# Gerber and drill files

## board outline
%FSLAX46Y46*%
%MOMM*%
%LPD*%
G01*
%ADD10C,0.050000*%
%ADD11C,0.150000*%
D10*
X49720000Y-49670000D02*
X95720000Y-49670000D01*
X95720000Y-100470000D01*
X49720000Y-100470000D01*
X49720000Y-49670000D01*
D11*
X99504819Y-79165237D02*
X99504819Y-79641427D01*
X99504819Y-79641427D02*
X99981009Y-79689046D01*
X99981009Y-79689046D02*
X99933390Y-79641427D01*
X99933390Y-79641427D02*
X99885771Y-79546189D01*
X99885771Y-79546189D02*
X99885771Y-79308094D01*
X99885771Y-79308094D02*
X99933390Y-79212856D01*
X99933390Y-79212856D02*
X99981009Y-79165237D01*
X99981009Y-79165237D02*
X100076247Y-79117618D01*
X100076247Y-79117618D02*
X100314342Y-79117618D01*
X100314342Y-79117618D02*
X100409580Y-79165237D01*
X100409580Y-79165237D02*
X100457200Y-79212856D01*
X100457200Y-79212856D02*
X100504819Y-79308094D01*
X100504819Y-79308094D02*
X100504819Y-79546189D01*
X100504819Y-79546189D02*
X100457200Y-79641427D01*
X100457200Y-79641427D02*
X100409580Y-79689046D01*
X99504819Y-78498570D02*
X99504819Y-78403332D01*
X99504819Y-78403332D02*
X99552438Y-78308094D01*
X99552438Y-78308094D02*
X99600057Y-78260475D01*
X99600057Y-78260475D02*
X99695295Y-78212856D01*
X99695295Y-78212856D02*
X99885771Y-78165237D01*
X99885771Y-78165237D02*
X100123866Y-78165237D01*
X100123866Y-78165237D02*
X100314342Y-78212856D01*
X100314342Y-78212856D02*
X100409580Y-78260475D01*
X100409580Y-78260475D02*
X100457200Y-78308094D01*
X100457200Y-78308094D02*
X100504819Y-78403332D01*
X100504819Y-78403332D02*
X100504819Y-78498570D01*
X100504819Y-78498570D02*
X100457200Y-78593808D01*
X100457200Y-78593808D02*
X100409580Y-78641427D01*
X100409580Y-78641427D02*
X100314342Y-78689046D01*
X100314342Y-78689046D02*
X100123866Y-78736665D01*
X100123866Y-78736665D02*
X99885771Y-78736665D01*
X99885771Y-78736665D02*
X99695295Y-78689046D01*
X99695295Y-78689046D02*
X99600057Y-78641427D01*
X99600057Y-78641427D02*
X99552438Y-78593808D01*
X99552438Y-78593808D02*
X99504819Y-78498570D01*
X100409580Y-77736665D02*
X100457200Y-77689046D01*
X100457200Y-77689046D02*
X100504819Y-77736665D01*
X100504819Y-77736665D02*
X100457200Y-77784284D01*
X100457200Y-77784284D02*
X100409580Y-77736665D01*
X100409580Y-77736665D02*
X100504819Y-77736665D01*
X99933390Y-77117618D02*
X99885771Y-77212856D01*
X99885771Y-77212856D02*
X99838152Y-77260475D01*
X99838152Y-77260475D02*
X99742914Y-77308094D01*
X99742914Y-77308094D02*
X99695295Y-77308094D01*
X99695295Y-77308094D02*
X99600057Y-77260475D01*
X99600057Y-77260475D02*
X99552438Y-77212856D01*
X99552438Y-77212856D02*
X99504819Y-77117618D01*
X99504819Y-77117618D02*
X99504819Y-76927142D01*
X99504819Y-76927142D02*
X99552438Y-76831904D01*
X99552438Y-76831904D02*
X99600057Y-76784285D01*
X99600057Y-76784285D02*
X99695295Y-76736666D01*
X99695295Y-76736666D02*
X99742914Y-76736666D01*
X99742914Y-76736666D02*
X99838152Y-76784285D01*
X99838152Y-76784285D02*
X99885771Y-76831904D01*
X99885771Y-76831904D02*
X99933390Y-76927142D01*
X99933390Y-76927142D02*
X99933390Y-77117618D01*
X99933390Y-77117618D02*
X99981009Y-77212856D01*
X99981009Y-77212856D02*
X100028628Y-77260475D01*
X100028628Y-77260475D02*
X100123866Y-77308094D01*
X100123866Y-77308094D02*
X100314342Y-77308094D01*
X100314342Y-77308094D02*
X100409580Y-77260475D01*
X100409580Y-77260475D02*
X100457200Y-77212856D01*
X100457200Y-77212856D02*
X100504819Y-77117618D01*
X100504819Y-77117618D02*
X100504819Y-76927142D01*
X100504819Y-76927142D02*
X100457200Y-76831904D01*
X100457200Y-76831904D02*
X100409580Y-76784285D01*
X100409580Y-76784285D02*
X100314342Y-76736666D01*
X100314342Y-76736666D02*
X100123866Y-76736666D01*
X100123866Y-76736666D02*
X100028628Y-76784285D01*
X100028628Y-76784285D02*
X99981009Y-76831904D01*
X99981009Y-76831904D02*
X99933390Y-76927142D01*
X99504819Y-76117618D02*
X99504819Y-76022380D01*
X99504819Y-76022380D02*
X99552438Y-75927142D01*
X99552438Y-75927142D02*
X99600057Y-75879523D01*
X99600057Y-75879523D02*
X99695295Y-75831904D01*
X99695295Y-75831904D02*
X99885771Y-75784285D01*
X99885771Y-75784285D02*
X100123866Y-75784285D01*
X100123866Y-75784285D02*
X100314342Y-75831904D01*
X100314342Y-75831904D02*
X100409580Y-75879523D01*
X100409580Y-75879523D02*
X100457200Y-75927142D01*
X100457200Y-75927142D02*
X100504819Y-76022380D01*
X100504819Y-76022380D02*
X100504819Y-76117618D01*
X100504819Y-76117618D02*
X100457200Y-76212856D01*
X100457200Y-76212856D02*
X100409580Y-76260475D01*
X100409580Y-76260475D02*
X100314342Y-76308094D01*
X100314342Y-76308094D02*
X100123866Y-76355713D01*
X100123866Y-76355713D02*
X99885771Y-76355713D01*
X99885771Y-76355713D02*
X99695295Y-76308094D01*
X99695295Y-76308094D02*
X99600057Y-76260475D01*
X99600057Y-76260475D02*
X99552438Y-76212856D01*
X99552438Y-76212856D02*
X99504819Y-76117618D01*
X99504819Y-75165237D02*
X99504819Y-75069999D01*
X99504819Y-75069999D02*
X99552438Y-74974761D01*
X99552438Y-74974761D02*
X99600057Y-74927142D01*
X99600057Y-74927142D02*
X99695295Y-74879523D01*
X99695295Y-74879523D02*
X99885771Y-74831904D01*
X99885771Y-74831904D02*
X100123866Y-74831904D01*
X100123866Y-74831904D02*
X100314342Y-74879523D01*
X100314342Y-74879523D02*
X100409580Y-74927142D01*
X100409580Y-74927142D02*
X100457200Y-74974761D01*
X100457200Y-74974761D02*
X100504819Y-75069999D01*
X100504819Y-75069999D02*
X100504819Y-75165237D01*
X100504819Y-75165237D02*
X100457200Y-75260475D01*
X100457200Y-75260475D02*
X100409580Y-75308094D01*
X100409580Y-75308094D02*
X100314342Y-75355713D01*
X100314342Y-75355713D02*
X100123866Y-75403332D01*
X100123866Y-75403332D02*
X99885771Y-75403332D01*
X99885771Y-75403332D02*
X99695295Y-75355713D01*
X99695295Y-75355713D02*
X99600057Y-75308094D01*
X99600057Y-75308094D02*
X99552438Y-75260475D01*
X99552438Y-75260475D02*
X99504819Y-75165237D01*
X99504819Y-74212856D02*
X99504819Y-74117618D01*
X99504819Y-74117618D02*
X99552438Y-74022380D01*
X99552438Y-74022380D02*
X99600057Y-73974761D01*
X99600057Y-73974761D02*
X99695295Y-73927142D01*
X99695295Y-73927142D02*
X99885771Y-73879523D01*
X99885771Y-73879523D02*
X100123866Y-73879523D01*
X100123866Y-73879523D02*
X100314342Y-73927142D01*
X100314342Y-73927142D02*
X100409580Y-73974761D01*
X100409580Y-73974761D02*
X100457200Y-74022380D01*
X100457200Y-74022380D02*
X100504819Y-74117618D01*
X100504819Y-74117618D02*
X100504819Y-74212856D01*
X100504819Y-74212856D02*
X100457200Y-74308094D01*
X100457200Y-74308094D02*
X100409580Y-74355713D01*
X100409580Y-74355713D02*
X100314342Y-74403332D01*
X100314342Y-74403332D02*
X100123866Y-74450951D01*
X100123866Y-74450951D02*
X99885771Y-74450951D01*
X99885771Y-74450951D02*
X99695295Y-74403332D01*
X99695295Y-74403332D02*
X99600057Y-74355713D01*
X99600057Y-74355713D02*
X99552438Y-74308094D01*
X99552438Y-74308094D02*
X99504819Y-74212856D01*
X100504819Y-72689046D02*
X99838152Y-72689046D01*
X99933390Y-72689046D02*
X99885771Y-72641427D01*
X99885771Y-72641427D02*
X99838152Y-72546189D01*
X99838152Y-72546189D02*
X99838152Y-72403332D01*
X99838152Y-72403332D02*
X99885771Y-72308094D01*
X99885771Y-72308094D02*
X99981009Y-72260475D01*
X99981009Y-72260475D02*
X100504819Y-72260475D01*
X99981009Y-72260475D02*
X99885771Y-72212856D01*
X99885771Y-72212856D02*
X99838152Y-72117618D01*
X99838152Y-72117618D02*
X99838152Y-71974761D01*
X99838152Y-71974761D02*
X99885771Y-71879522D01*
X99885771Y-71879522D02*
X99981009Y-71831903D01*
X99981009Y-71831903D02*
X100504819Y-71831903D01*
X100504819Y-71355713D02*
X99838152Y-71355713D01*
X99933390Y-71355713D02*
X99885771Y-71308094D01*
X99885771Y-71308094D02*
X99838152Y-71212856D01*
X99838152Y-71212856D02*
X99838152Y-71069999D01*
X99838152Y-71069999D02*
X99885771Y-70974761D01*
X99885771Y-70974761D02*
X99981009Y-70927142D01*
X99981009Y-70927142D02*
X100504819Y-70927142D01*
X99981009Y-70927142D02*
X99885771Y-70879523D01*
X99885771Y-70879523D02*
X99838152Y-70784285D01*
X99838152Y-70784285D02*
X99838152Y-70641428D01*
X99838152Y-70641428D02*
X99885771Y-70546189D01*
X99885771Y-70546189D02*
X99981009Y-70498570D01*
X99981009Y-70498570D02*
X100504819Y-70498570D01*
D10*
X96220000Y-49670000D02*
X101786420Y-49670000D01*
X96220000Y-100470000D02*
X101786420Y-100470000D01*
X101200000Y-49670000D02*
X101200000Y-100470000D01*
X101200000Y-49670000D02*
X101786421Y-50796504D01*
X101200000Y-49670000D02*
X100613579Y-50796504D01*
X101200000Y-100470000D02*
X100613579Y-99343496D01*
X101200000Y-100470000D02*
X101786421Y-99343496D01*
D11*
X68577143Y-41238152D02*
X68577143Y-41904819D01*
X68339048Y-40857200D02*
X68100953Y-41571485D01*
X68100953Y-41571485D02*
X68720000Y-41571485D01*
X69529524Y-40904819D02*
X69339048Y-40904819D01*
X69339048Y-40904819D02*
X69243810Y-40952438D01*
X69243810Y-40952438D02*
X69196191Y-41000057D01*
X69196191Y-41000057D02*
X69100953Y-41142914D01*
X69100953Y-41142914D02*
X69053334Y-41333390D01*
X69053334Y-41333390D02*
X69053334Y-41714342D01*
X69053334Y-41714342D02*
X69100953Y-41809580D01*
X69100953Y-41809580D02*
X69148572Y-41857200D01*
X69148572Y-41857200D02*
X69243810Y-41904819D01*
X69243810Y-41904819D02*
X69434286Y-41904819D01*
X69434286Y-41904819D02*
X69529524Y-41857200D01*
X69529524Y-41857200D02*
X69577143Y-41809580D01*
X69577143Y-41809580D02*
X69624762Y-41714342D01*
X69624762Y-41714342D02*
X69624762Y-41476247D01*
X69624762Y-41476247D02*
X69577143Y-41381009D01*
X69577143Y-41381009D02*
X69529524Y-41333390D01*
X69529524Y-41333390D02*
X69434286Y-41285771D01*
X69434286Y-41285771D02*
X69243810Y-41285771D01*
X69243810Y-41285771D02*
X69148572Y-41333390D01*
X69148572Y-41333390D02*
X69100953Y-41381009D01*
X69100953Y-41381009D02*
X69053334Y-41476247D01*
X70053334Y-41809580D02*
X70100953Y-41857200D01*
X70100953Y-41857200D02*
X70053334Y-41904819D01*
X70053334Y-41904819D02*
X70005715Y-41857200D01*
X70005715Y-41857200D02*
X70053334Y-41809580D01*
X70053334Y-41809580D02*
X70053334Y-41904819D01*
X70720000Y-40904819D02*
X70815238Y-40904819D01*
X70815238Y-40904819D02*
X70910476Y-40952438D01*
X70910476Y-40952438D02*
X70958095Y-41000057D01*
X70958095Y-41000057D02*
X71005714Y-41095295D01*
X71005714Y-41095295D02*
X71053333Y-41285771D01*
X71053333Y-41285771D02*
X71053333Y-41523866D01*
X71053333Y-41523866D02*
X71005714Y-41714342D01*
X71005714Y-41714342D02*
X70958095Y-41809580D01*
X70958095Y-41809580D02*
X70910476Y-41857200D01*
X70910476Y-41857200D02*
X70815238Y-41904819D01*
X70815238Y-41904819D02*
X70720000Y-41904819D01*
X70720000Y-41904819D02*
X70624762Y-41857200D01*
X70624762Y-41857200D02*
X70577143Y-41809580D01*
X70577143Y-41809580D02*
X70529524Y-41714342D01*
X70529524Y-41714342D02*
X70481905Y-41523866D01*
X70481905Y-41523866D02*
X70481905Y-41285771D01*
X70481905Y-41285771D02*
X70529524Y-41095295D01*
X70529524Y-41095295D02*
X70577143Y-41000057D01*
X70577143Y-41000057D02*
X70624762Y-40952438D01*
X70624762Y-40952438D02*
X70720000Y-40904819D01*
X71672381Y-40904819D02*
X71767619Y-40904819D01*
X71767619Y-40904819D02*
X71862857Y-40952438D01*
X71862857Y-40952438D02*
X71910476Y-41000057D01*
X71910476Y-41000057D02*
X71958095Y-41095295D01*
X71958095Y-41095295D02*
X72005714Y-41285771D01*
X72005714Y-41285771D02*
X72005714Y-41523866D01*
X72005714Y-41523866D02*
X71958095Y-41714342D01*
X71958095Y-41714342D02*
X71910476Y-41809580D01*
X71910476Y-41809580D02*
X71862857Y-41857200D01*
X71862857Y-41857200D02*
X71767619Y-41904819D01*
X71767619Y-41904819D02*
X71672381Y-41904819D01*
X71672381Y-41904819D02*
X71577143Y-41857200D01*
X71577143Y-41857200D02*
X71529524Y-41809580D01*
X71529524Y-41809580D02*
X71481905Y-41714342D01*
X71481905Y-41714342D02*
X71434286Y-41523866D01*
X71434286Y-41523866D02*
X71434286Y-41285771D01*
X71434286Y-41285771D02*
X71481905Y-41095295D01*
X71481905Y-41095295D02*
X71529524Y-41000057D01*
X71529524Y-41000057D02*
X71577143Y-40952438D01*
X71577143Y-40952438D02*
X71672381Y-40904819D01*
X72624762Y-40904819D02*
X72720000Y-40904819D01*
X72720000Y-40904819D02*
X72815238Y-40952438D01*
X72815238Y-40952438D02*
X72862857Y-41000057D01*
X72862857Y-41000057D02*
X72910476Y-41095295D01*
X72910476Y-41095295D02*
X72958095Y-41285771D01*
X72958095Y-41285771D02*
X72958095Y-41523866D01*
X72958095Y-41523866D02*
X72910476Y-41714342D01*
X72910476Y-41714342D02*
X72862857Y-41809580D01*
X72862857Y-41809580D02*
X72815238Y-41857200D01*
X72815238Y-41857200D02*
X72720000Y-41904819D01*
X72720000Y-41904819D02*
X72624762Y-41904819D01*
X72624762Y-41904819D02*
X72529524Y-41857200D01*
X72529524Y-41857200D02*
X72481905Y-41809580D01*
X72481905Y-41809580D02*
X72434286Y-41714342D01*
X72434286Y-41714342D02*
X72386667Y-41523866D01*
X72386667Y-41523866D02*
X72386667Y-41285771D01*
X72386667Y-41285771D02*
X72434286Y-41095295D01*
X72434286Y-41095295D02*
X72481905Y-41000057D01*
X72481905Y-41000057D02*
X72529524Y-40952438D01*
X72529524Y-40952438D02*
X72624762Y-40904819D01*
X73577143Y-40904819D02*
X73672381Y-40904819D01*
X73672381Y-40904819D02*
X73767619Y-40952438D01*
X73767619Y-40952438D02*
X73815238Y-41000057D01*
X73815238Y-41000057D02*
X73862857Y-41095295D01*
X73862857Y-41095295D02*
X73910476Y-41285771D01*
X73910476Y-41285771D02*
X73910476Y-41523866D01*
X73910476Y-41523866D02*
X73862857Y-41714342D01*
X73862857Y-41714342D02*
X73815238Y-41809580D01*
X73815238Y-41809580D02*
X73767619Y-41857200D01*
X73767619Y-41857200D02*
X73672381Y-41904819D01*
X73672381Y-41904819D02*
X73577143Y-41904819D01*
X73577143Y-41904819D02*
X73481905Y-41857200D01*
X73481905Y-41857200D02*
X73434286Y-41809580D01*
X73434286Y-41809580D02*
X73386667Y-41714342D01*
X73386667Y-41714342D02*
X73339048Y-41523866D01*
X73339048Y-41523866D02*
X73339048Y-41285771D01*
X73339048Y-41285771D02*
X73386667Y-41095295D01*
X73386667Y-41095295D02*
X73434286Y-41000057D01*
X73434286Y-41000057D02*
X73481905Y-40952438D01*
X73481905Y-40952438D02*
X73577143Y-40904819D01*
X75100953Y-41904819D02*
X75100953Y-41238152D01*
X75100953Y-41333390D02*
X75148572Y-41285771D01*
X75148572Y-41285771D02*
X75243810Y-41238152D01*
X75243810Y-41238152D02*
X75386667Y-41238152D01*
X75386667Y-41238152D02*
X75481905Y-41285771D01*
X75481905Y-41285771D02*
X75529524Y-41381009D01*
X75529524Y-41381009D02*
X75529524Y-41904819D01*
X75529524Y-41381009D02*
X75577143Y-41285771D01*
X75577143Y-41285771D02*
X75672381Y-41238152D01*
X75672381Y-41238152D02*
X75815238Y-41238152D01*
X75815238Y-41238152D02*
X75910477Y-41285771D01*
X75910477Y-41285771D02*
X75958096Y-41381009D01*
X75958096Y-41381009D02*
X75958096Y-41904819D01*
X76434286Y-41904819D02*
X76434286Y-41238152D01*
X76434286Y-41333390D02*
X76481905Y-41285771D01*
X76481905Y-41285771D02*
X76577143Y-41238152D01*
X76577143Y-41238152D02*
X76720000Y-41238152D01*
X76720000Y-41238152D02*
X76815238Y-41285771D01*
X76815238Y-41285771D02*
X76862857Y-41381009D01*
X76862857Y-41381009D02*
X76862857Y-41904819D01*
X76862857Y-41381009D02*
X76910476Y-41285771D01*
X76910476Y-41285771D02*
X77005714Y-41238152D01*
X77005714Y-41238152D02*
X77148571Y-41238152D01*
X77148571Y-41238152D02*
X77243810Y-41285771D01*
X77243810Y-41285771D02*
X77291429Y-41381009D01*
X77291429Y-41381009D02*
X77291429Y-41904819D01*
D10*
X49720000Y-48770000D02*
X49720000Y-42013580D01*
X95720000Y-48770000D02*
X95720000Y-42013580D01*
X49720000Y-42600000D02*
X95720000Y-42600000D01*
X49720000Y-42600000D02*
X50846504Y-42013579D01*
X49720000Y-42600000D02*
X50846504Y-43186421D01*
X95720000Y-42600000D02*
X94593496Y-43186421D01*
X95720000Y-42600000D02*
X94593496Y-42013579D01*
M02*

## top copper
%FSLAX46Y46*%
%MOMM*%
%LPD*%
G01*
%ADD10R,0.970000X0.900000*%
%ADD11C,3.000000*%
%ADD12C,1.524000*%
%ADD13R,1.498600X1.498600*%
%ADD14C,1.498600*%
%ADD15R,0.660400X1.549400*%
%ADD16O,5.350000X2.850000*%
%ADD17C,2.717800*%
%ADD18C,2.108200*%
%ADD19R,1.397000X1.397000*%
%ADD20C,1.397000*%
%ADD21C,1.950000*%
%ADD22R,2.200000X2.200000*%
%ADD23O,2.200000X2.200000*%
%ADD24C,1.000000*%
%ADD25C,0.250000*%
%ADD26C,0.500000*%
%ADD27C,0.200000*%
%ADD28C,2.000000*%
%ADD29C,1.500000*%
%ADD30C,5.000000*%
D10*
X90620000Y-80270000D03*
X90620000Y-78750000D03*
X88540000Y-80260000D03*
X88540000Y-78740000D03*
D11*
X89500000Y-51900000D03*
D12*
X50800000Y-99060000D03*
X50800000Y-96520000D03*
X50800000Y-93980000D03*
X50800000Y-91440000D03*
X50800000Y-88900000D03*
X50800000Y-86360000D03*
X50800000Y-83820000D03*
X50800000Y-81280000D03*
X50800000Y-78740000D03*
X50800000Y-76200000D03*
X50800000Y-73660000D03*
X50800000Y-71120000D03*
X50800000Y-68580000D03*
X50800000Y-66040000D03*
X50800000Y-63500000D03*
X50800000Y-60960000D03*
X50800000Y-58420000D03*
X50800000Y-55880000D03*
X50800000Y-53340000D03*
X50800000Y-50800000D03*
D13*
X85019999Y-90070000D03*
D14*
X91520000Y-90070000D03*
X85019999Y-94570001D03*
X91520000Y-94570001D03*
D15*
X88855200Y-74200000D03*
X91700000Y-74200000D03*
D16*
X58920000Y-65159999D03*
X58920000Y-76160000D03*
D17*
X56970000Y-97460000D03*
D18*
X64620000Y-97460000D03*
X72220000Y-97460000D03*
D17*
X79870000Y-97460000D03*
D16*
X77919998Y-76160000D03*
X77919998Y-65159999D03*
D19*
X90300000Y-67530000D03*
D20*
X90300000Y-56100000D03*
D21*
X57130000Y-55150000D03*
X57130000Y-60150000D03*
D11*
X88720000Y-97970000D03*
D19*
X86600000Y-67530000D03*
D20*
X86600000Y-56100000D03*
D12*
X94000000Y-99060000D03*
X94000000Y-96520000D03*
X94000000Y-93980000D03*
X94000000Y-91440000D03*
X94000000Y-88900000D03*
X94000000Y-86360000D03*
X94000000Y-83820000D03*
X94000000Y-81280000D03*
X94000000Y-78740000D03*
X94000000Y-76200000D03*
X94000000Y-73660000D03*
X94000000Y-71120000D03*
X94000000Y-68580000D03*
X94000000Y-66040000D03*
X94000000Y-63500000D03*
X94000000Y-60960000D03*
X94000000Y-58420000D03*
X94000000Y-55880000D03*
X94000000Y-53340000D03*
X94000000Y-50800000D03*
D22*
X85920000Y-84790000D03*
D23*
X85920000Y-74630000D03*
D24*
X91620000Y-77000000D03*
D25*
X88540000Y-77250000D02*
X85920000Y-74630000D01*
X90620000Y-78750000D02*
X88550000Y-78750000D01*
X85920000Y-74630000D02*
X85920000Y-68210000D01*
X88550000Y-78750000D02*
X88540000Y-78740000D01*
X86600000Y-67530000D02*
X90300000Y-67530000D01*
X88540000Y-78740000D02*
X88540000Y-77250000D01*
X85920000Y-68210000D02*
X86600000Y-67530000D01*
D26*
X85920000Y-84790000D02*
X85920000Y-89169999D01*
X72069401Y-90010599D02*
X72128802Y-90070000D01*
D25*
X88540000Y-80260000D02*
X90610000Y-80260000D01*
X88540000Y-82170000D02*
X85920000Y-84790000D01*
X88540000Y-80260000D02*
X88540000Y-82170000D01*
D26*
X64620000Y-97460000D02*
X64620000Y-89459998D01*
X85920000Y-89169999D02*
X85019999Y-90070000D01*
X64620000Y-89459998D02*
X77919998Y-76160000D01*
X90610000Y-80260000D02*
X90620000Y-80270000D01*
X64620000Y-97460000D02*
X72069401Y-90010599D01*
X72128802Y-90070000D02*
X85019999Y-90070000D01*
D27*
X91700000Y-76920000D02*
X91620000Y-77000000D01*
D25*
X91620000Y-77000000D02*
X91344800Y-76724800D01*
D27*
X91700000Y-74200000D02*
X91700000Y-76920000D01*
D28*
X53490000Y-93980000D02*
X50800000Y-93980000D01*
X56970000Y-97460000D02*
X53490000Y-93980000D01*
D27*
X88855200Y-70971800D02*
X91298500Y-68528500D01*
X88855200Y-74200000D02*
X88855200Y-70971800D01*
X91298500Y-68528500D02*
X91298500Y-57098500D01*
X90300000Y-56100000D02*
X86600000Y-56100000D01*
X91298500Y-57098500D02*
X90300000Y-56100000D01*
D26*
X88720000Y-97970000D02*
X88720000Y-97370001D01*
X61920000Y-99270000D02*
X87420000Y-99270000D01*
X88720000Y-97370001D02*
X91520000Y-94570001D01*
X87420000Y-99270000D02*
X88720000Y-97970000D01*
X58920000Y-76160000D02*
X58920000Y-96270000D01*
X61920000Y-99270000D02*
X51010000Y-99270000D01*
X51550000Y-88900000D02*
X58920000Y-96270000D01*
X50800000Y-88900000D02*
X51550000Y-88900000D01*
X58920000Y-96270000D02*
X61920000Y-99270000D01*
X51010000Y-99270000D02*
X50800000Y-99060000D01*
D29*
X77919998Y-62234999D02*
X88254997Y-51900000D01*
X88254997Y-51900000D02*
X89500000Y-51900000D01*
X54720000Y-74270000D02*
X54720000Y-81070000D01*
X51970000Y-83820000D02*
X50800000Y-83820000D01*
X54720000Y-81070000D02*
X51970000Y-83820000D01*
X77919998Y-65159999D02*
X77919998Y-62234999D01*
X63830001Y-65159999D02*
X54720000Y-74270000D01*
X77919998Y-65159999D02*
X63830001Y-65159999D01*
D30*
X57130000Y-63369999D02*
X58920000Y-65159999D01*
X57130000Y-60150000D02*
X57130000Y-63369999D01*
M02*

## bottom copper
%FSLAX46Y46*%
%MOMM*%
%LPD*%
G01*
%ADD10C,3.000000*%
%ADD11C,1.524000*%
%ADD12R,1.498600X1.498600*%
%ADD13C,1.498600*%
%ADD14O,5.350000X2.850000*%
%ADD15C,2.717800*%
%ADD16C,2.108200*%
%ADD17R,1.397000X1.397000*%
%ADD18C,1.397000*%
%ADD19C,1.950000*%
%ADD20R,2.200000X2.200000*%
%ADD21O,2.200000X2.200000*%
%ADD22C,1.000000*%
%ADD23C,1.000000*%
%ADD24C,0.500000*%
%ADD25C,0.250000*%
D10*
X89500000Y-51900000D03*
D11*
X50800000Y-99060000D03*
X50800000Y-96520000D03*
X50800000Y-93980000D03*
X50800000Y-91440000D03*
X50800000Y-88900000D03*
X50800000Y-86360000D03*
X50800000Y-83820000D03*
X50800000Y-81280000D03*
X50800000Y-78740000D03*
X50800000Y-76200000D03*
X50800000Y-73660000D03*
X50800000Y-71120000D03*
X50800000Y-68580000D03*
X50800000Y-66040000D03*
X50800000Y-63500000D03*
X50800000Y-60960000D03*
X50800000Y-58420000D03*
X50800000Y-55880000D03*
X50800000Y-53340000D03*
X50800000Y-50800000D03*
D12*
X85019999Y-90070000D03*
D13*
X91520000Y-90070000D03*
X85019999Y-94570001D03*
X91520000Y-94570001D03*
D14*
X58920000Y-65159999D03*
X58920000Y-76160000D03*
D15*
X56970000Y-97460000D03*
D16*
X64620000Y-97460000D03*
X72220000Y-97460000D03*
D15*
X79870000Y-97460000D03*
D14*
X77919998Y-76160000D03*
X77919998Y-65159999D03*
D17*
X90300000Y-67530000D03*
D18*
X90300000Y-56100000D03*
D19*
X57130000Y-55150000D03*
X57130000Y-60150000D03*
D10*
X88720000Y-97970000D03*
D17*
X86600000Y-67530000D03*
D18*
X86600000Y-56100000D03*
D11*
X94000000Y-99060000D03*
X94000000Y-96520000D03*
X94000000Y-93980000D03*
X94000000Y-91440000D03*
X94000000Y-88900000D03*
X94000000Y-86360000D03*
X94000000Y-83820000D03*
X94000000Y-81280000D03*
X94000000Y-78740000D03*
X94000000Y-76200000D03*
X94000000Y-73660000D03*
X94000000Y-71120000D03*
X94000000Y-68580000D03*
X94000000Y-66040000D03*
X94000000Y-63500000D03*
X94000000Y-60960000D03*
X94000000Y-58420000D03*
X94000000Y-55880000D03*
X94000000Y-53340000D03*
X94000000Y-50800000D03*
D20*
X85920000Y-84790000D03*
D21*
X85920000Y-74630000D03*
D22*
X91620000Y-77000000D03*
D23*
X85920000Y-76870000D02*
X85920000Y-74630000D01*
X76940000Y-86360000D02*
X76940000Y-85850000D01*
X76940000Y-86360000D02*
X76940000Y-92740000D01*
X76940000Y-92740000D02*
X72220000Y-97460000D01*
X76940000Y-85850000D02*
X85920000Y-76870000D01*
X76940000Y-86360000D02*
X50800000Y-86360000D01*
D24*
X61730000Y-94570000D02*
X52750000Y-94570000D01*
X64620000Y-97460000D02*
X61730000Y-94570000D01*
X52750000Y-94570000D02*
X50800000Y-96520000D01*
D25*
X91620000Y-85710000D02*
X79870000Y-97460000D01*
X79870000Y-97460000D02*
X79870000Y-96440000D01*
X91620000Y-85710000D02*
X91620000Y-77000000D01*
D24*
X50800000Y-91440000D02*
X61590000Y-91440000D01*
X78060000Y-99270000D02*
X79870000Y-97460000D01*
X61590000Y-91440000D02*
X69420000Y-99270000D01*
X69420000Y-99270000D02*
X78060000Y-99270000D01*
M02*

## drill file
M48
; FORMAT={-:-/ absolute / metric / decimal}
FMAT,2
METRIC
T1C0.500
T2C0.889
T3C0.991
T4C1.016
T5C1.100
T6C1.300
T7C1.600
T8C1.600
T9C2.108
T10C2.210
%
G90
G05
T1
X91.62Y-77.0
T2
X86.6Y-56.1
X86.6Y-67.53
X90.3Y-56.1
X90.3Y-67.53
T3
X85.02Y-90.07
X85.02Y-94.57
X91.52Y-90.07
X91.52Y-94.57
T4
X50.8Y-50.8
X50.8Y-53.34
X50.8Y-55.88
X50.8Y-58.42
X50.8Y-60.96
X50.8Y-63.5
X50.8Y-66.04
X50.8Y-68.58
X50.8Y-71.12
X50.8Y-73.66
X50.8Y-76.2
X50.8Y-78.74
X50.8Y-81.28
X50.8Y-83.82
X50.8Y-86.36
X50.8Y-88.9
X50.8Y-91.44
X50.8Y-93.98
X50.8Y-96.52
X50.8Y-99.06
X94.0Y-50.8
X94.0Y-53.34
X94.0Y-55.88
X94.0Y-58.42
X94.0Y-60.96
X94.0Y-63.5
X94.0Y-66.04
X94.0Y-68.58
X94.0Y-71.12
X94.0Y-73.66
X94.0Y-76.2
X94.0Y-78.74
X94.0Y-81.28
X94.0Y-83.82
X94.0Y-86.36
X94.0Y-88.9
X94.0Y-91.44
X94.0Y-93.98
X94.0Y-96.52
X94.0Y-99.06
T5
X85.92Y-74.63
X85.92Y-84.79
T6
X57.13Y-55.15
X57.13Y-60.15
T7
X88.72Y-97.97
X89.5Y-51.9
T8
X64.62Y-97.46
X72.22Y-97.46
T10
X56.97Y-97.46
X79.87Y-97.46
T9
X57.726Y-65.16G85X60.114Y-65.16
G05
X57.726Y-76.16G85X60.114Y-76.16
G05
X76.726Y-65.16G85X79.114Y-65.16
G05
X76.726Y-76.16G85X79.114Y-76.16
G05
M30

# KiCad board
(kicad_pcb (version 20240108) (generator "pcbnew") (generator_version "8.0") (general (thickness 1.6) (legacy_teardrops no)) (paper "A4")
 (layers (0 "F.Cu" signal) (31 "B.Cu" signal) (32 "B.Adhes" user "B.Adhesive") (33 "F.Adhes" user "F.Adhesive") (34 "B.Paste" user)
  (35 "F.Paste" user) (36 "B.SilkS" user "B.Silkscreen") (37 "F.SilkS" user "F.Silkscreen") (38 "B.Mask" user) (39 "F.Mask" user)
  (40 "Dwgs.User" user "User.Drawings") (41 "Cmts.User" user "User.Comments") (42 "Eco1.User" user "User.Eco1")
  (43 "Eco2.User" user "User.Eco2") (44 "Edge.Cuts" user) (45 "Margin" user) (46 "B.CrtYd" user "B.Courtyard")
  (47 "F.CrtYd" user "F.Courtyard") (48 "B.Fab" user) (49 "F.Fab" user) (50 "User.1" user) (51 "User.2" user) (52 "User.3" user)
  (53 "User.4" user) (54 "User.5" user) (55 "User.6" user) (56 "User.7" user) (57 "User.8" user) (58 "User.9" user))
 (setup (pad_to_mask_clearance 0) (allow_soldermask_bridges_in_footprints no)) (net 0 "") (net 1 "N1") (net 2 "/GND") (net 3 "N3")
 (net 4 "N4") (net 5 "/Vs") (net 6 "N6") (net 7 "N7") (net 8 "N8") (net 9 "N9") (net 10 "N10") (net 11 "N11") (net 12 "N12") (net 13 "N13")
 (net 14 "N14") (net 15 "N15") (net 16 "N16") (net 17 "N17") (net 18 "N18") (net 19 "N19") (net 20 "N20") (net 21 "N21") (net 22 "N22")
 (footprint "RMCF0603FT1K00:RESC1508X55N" (layer "F.Cu") (at 90.62 79.51 90)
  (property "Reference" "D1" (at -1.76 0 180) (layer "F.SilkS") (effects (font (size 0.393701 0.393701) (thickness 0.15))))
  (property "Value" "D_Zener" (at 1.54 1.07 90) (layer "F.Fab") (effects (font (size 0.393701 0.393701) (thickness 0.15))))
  (pad "1" smd rect (at -0.76 0 90) (size 0.9 0.97) (layers "F.Cu" "F.Paste" "F.Mask") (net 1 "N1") (solder_mask_margin 0.102))
  (pad "2" smd rect (at 0.76 0 90) (size 0.9 0.97) (layers "F.Cu" "F.Paste" "F.Mask") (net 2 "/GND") (solder_mask_margin 0.102)))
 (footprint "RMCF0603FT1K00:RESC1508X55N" (layer "F.Cu") (at 88.54 79.5 90)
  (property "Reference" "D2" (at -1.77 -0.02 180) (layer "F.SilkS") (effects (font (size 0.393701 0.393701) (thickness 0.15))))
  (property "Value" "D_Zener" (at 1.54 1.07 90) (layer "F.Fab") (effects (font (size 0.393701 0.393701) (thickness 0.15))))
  (pad "1" smd rect (at -0.76 0 90) (size 0.9 0.97) (layers "F.Cu" "F.Paste" "F.Mask") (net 1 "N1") (solder_mask_margin 0.102))
  (pad "2" smd rect (at 0.76 0 90) (size 0.9 0.97) (layers "F.Cu" "F.Paste" "F.Mask") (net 2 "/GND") (solder_mask_margin 0.102)))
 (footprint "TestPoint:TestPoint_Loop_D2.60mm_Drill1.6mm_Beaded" (layer "F.Cu") (at 89.5 51.9)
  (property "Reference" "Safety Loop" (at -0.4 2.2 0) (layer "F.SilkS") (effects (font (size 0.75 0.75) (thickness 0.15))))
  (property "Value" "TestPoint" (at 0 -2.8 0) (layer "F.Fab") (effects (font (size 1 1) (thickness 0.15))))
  (pad "1" thru_hole circle (at 0 0) (size 3 3) (drill 1.6) (layers "*.Cu" "*.Mask") (remove_unused_layers no) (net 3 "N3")))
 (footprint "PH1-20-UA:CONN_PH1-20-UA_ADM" (layer "F.Cu") (at 50.8 99.06 90)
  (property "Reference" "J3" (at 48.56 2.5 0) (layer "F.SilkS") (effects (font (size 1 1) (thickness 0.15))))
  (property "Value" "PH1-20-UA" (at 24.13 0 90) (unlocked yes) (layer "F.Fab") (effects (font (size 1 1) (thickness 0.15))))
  (pad "1" thru_hole circle (at 0 0 90) (size 1.524 1.524) (drill 1.016) (layers "*.Cu" "*.Mask") (remove_unused_layers no) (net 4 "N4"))
  (pad "2" thru_hole circle (at 2.54 0 90) (size 1.524 1.524) (drill 1.016) (layers "*.Cu" "*.Mask") (remove_unused_layers no) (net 1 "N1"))
  (pad "3" thru_hole circle (at 5.08 0 90) (size 1.524 1.524) (drill 1.016) (layers "*.Cu" "*.Mask") (remove_unused_layers no) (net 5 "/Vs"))
  (pad "4" thru_hole circle (at 7.62 0 90) (size 1.524 1.524) (drill 1.016) (layers "*.Cu" "*.Mask") (remove_unused_layers no) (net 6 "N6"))
  (pad "5" thru_hole circle (at 10.16 0 90) (size 1.524 1.524) (drill 1.016) (layers "*.Cu" "*.Mask") (remove_unused_layers no) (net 4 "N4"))
  (pad "6" thru_hole circle (at 12.7 0 90) (size 1.524 1.524) (drill 1.016) (layers "*.Cu" "*.Mask") (remove_unused_layers no)
   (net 2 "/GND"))
  (pad "7" thru_hole circle (at 15.24 0 90) (size 1.524 1.524) (drill 1.016) (layers "*.Cu" "*.Mask") (remove_unused_layers no) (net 3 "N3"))
  (pad "8" thru_hole circle (at 17.78 0 90) (size 1.524 1.524) (drill 1.016) (layers "*.Cu" "*.Mask") (remove_unused_layers no) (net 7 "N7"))
  (pad "9" thru_hole circle (at 20.32 0 90) (size 1.524 1.524) (drill 1.016) (layers "*.Cu" "*.Mask") (remove_unused_layers no) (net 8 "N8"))
  (pad "10" thru_hole circle (at 22.86 0 90) (size 1.524 1.524) (drill 1.016) (layers "*.Cu" "*.Mask") (remove_unused_layers no)
   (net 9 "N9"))
  (pad "11" thru_hole circle (at 25.4 0 90) (size 1.524 1.524) (drill 1.016) (layers "*.Cu" "*.Mask") (remove_unused_layers no)
   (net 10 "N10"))
  (pad "12" thru_hole circle (at 27.94 0 90) (size 1.524 1.524) (drill 1.016) (layers "*.Cu" "*.Mask") (remove_unused_layers no)
   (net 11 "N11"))
  (pad "13" thru_hole circle (at 30.48 0 90) (size 1.524 1.524) (drill 1.016) (layers "*.Cu" "*.Mask") (remove_unused_layers no)
   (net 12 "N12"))
  (pad "14" thru_hole circle (at 33.02 0 90) (size 1.524 1.524) (drill 1.016) (layers "*.Cu" "*.Mask") (remove_unused_layers no)
   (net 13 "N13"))
  (pad "15" thru_hole circle (at 35.56 0 90) (size 1.524 1.524) (drill 1.016) (layers "*.Cu" "*.Mask") (remove_unused_layers no)
   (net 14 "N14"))
  (pad "16" thru_hole circle (at 38.1 0 90) (size 1.524 1.524) (drill 1.016) (layers "*.Cu" "*.Mask") (remove_unused_layers no)
   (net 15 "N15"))
  (pad "17" thru_hole circle (at 40.64 0 90) (size 1.524 1.524) (drill 1.016) (layers "*.Cu" "*.Mask") (remove_unused_layers no)
   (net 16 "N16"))
  (pad "18" thru_hole circle (at 43.18 0 90) (size 1.524 1.524) (drill 1.016) (layers "*.Cu" "*.Mask") (remove_unused_layers no)
   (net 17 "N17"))
  (pad "19" thru_hole circle (at 45.72 0 90) (size 1.524 1.524) (drill 1.016) (layers "*.Cu" "*.Mask") (remove_unused_layers no)
   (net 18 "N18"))
  (pad "20" thru_hole circle (at 48.26 0 90) (size 1.524 1.524) (drill 1.016) (layers "*.Cu" "*.Mask") (remove_unused_layers no)
   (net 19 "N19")))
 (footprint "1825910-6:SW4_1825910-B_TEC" (layer "F.Cu") (at 91.52 94.570001)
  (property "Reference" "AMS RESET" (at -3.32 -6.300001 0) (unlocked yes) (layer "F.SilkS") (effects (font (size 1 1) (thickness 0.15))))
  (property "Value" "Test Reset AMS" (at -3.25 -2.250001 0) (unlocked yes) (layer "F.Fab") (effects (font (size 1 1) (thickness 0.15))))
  (pad "1" thru_hole rect (at -6.500001 -4.500001) (size 1.4986 1.4986) (drill 0.9906) (layers "*.Cu" "*.Mask") (remove_unused_layers no)
   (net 1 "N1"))
  (pad "2" thru_hole circle (at 0 -4.500001) (size 1.4986 1.4986) (drill 0.9906) (layers "*.Cu" "*.Mask") (remove_unused_layers no))
  (pad "3" thru_hole circle (at -6.500001 0) (size 1.4986 1.4986) (drill 0.9906) (layers "*.Cu" "*.Mask") (remove_unused_layers no))
  (pad "4" thru_hole circle (at 0 0) (size 1.4986 1.4986) (drill 0.9906) (layers "*.Cu" "*.Mask") (remove_unused_layers no) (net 4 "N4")))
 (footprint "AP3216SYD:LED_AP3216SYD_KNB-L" (layer "F.Cu") (at 90.2776 74.2)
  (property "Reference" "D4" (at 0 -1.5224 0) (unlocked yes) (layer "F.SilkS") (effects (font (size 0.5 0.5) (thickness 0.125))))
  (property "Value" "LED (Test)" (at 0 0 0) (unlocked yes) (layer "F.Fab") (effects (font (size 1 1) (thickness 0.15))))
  (pad "1" smd rect (at -1.4224 0) (size 0.6604 1.5494) (layers "F.Cu" "F.Paste" "F.Mask") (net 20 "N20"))
  (pad "2" smd rect (at 1.4224 0) (size 0.6604 1.5494) (layers "F.Cu" "F.Paste" "F.Mask") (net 6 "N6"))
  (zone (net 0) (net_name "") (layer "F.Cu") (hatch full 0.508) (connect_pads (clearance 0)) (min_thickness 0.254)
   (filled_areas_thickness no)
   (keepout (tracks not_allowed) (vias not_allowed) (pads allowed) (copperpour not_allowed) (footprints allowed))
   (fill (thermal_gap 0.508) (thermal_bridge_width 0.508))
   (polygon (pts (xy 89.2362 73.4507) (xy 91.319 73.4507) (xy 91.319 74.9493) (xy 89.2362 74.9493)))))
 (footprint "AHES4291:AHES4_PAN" (layer "F.Cu") (at 58.919999 65.159998)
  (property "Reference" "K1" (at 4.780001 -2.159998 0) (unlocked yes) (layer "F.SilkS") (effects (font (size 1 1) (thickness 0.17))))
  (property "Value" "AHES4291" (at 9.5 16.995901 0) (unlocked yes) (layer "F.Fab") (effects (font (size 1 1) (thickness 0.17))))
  (pad "1" thru_hole oval (at 0.000001 0.000001) (size 5.35 2.85) (drill oval 4.4958 2.1082) (layers "*.Cu" "*.Mask")
   (remove_unused_layers no) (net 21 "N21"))
  (pad "2" thru_hole oval (at 0.000001 11.000002) (size 5.35 2.85) (drill oval 4.4958 2.1082) (layers "*.Cu" "*.Mask")
   (remove_unused_layers no) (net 4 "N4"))
  (pad "3" thru_hole circle (at -1.949999 32.300002) (size 2.7178 2.7178) (drill 2.2098) (layers "*.Cu" "*.Mask") (remove_unused_layers no)
   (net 5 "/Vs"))
  (pad "4" thru_hole circle (at 5.700001 32.300002) (size 2.1082 2.1082) (drill 1.6002) (layers "*.Cu" "*.Mask") (remove_unused_layers no)
   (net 1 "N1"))
  (pad "5" thru_hole circle (at 13.300001 32.300002) (size 2.1082 2.1082) (drill 1.6002) (layers "*.Cu" "*.Mask") (remove_unused_layers no)
   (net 2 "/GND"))
  (pad "6" thru_hole circle (at 20.950001 32.300002) (size 2.7178 2.7178) (drill 2.2098) (layers "*.Cu" "*.Mask") (remove_unused_layers no)
   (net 6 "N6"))
  (pad "7" thru_hole oval (at 18.999999 11.000002) (size 5.35 2.85) (drill oval 4.4958 2.1082) (layers "*.Cu" "*.Mask")
   (remove_unused_layers no) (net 1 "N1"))
  (pad "8" thru_hole oval (at 18.999999 0.000001) (size 5.35 2.85) (drill oval 4.4958 2.1082) (layers "*.Cu" "*.Mask")
   (remove_unused_layers no) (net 3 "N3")))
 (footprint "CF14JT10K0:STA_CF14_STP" (layer "F.Cu") (at 90.3 67.53 90)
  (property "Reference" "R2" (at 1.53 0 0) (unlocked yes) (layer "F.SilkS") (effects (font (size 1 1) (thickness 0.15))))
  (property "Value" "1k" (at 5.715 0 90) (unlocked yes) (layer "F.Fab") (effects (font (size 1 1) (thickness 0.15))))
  (pad "1" thru_hole rect (at 0 0 90) (size 1.397 1.397) (drill 0.889) (layers "*.Cu" "*.Mask") (remove_unused_layers no) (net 2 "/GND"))
  (pad "2" thru_hole circle (at 11.43 0 90) (size 1.397 1.397) (drill 0.889) (layers "*.Cu" "*.Mask") (remove_unused_layers no)
   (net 20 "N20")))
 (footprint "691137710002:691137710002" (layer "F.Cu") (at 57.13 57.65 -90)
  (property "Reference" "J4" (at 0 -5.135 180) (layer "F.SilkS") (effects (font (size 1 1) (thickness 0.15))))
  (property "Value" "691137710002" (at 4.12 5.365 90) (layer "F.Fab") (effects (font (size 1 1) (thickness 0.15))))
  (pad "1" thru_hole circle (at -2.5 0 270) (size 1.95 1.95) (drill 1.3) (layers "*.Cu" "*.Mask") (remove_unused_layers no) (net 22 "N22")
   (solder_mask_margin 0.102))
  (pad "2" thru_hole circle (at 2.5 0 270) (size 1.95 1.95) (drill 1.3) (layers "*.Cu" "*.Mask") (remove_unused_layers no) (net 21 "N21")
   (solder_mask_margin 0.102)))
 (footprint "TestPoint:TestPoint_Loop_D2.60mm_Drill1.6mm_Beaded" (layer "F.Cu") (at 88.72 97.97)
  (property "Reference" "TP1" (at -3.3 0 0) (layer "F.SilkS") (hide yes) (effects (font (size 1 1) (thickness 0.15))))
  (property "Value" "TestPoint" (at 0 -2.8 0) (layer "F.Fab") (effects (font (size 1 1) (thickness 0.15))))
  (pad "1" thru_hole circle (at 0 0) (size 3 3) (drill 1.6) (layers "*.Cu" "*.Mask") (remove_unused_layers no) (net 4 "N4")))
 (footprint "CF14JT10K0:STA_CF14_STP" (layer "F.Cu") (at 86.6 67.53 90)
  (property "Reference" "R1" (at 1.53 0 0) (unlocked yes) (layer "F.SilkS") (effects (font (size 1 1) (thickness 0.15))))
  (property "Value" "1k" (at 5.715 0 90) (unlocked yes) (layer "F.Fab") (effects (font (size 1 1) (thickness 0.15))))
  (pad "1" thru_hole rect (at 0 0 90) (size 1.397 1.397) (drill 0.889) (layers "*.Cu" "*.Mask") (remove_unused_layers no) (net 2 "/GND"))
  (pad "2" thru_hole circle (at 11.43 0 90) (size 1.397 1.397) (drill 0.889) (layers "*.Cu" "*.Mask") (remove_unused_layers no)
   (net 20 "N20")))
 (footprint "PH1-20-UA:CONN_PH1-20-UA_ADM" (layer "F.Cu") (at 94 99.06 90)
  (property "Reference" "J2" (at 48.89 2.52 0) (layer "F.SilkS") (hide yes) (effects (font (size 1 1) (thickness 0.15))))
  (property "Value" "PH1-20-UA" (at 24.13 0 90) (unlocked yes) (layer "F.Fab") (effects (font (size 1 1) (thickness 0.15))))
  (pad "1" thru_hole circle (at 0 0 90) (size 1.524 1.524) (drill 1.016) (layers "*.Cu" "*.Mask") (remove_unused_layers no))
  (pad "2" thru_hole circle (at 2.54 0 90) (size 1.524 1.524) (drill 1.016) (layers "*.Cu" "*.Mask") (remove_unused_layers no))
  (pad "3" thru_hole circle (at 5.08 0 90) (size 1.524 1.524) (drill 1.016) (layers "*.Cu" "*.Mask") (remove_unused_layers no))
  (pad "4" thru_hole circle (at 7.62 0 90) (size 1.524 1.524) (drill 1.016) (layers "*.Cu" "*.Mask") (remove_unused_layers no))
  (pad "5" thru_hole circle (at 10.16 0 90) (size 1.524 1.524) (drill 1.016) (layers "*.Cu" "*.Mask") (remove_unused_layers no))
  (pad "6" thru_hole circle (at 12.7 0 90) (size 1.524 1.524) (drill 1.016) (layers "*.Cu" "*.Mask") (remove_unused_layers no))
  (pad "7" thru_hole circle (at 15.24 0 90) (size 1.524 1.524) (drill 1.016) (layers "*.Cu" "*.Mask") (remove_unused_layers no))
  (pad "8" thru_hole circle (at 17.78 0 90) (size 1.524 1.524) (drill 1.016) (layers "*.Cu" "*.Mask") (remove_unused_layers no))
  (pad "9" thru_hole circle (at 20.32 0 90) (size 1.524 1.524) (drill 1.016) (layers "*.Cu" "*.Mask") (remove_unused_layers no))
  (pad "10" thru_hole circle (at 22.86 0 90) (size 1.524 1.524) (drill 1.016) (layers "*.Cu" "*.Mask") (remove_unused_layers no))
  (pad "11" thru_hole circle (at 25.4 0 90) (size 1.524 1.524) (drill 1.016) (layers "*.Cu" "*.Mask") (remove_unused_layers no))
  (pad "12" thru_hole circle (at 27.94 0 90) (size 1.524 1.524) (drill 1.016) (layers "*.Cu" "*.Mask") (remove_unused_layers no))
  (pad "13" thru_hole circle (at 30.48 0 90) (size 1.524 1.524) (drill 1.016) (layers "*.Cu" "*.Mask") (remove_unused_layers no))
  (pad "14" thru_hole circle (at 33.02 0 90) (size 1.524 1.524) (drill 1.016) (layers "*.Cu" "*.Mask") (remove_unused_layers no))
  (pad "15" thru_hole circle (at 35.56 0 90) (size 1.524 1.524) (drill 1.016) (layers "*.Cu" "*.Mask") (remove_unused_layers no))
  (pad "16" thru_hole circle (at 38.1 0 90) (size 1.524 1.524) (drill 1.016) (layers "*.Cu" "*.Mask") (remove_unused_layers no))
  (pad "17" thru_hole circle (at 40.64 0 90) (size 1.524 1.524) (drill 1.016) (layers "*.Cu" "*.Mask") (remove_unused_layers no))
  (pad "18" thru_hole circle (at 43.18 0 90) (size 1.524 1.524) (drill 1.016) (layers "*.Cu" "*.Mask") (remove_unused_layers no))
  (pad "19" thru_hole circle (at 45.72 0 90) (size 1.524 1.524) (drill 1.016) (layers "*.Cu" "*.Mask") (remove_unused_layers no))
  (pad "20" thru_hole circle (at 48.26 0 90) (size 1.524 1.524) (drill 1.016) (layers "*.Cu" "*.Mask") (remove_unused_layers no)))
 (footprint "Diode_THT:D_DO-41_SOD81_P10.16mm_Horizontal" (layer "F.Cu") (at 85.92 84.79 90)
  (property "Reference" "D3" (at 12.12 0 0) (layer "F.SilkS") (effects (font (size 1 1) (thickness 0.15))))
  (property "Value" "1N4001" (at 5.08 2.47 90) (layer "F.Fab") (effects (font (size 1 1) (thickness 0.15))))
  (pad "1" thru_hole rect (at 0 0 90) (size 2.2 2.2) (drill 1.1) (layers "*.Cu" "*.Mask") (remove_unused_layers no) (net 1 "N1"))
  (pad "2" thru_hole oval (at 10.16 0 90) (size 2.2 2.2) (drill 1.1) (layers "*.Cu" "*.Mask") (remove_unused_layers no) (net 2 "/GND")))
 (gr_rect (start 49.72 49.67) (end 95.72 100.47) (stroke (width 0.05) (type default)) (fill none) (layer "Edge.Cuts"))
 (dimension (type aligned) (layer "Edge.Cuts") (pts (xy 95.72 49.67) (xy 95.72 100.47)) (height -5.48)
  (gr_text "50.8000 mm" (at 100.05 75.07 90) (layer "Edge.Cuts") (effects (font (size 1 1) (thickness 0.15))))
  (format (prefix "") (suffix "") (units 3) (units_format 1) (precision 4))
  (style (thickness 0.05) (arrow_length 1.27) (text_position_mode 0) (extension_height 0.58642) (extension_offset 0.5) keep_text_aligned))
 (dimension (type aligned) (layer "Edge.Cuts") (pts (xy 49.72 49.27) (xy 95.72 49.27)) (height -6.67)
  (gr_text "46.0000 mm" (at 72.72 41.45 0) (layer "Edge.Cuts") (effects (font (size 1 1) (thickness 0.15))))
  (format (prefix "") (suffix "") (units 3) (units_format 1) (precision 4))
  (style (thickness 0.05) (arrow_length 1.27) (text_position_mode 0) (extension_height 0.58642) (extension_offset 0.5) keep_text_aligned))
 (segment (start 88.54 77.25) (end 85.92 74.63) (width 0.25) (layer "F.Cu") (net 2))
 (segment (start 90.62 78.75) (end 88.55 78.75) (width 0.25) (layer "F.Cu") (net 2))
 (segment (start 85.92 74.63) (end 85.92 68.21) (width 0.25) (layer "F.Cu") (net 2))
 (segment (start 88.55 78.75) (end 88.54 78.74) (width 0.25) (layer "F.Cu") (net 2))
 (segment (start 86.6 67.53) (end 90.3 67.53) (width 0.25) (layer "F.Cu") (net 2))
 (segment (start 88.54 78.74) (end 88.54 77.25) (width 0.25) (layer "F.Cu") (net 2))
 (segment (start 85.92 68.21) (end 86.6 67.53) (width 0.25) (layer "F.Cu") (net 2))
 (segment (start 85.92 76.87) (end 85.92 74.63) (width 1) (layer "B.Cu") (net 2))
 (segment (start 76.94 86.36) (end 76.94 85.85) (width 1) (layer "B.Cu") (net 2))
 (segment (start 76.94 86.36) (end 76.94 92.74) (width 1) (layer "B.Cu") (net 2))
 (segment (start 76.94 92.74) (end 72.22 97.46) (width 1) (layer "B.Cu") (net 2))
 (segment (start 76.94 85.85) (end 85.92 76.87) (width 1) (layer "B.Cu") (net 2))
 (segment (start 76.94 86.36) (end 50.8 86.36) (width 1) (layer "B.Cu") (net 2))
 (segment (start 85.92 84.79) (end 85.92 89.169999) (width 0.5) (layer "F.Cu") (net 1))
 (segment (start 72.069401 90.010599) (end 72.128802 90.07) (width 0.5) (layer "F.Cu") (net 1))
 (segment (start 88.54 80.26) (end 90.61 80.26) (width 0.25) (layer "F.Cu") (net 1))
 (segment (start 88.54 82.17) (end 85.92 84.79) (width 0.25) (layer "F.Cu") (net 1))
 (segment (start 88.54 80.26) (end 88.54 82.17) (width 0.25) (layer "F.Cu") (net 1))
 (segment (start 64.62 97.46) (end 64.62 89.459998) (width 0.5) (layer "F.Cu") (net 1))
 (segment (start 85.92 89.169999) (end 85.019999 90.07) (width 0.5) (layer "F.Cu") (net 1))
 (segment (start 64.62 89.459998) (end 77.919998 76.16) (width 0.5) (layer "F.Cu") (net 1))
 (segment (start 90.61 80.26) (end 90.62 80.27) (width 0.5) (layer "F.Cu") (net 1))
 (segment (start 64.62 97.46) (end 72.069401 90.010599) (width 0.5) (layer "F.Cu") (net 1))
 (segment (start 72.128802 90.07) (end 85.019999 90.07) (width 0.5) (layer "F.Cu") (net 1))
 (segment (start 61.73 94.57) (end 52.75 94.57) (width 0.5) (layer "B.Cu") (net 1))
 (segment (start 64.62 97.46) (end 61.73 94.57) (width 0.5) (layer "B.Cu") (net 1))
 (segment (start 52.75 94.57) (end 50.8 96.52) (width 0.5) (layer "B.Cu") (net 1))
 (segment (start 91.7 76.92) (end 91.62 77) (width 0.2) (layer "F.Cu") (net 6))
 (segment (start 91.62 77) (end 91.3448 76.7248) (width 0.25) (layer "F.Cu") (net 6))
 (segment (start 91.7 74.2) (end 91.7 76.92) (width 0.2) (layer "F.Cu") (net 6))
 (via (at 91.62 77) (size 1) (drill 0.5) (layers "F.Cu" "B.Cu") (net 6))
 (segment (start 91.62 85.71) (end 79.87 97.46) (width 0.25) (layer "B.Cu") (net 6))
 (segment (start 79.87 97.46) (end 79.87 96.44) (width 0.25) (layer "B.Cu") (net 6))
 (segment (start 91.62 85.71) (end 91.62 77) (width 0.25) (layer "B.Cu") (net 6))
 (segment (start 50.8 91.44) (end 61.59 91.44) (width 0.5) (layer "B.Cu") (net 6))
 (segment (start 78.06 99.27) (end 79.87 97.46) (width 0.5) (layer "B.Cu") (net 6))
 (segment (start 61.59 91.44) (end 69.42 99.27) (width 0.5) (layer "B.Cu") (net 6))
 (segment (start 69.42 99.27) (end 78.06 99.27) (width 0.5) (layer "B.Cu") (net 6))
 (segment (start 53.49 93.98) (end 50.8 93.98) (width 2) (layer "F.Cu") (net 5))
 (segment (start 56.97 97.46) (end 53.49 93.98) (width 2) (layer "F.Cu") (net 5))
 (segment (start 88.8552 70.9718) (end 91.2985 68.5285) (width 0.2) (layer "F.Cu") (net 20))
 (segment (start 88.8552 74.2) (end 88.8552 70.9718) (width 0.2) (layer "F.Cu") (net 20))
 (segment (start 91.2985 68.5285) (end 91.2985 57.0985) (width 0.2) (layer "F.Cu") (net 20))
 (segment (start 90.3 56.1) (end 86.6 56.1) (width 0.2) (layer "F.Cu") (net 20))
 (segment (start 91.2985 57.0985) (end 90.3 56.1) (width 0.2) (layer "F.Cu") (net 20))
 (segment (start 88.72 97.97) (end 88.72 97.370001) (width 0.5) (layer "F.Cu") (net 4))
 (segment (start 61.92 99.27) (end 87.42 99.27) (width 0.5) (layer "F.Cu") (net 4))
 (segment (start 88.72 97.370001) (end 91.52 94.570001) (width 0.5) (layer "F.Cu") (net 4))
 (segment (start 87.42 99.27) (end 88.72 97.97) (width 0.5) (layer "F.Cu") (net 4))
 (segment (start 58.92 76.16) (end 58.92 96.27) (width 0.5) (layer "F.Cu") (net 4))
 (segment (start 61.92 99.27) (end 51.01 99.27) (width 0.5) (layer "F.Cu") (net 4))
 (segment (start 51.55 88.9) (end 58.92 96.27) (width 0.5) (layer "F.Cu") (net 4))
 (segment (start 50.8 88.9) (end 51.55 88.9) (width 0.5) (layer "F.Cu") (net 4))
 (segment (start 58.92 96.27) (end 61.92 99.27) (width 0.5) (layer "F.Cu") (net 4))
 (segment (start 51.01 99.27) (end 50.8 99.06) (width 0.5) (layer "F.Cu") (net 4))
 (segment (start 77.919998 62.234999) (end 88.254997 51.9) (width 1.5) (layer "F.Cu") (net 3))
 (segment (start 88.254997 51.9) (end 89.5 51.9) (width 1.5) (layer "F.Cu") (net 3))
 (segment (start 54.72 74.27) (end 54.72 81.07) (width 1.5) (layer "F.Cu") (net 3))
 (segment (start 51.97 83.82) (end 50.8 83.82) (width 1.5) (layer "F.Cu") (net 3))
 (segment (start 54.72 81.07) (end 51.97 83.82) (width 1.5) (layer "F.Cu") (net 3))
 (segment (start 77.919998 65.159999) (end 77.919998 62.234999) (width 1.5) (layer "F.Cu") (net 3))
 (segment (start 63.830001 65.159999) (end 54.72 74.27) (width 1.5) (layer "F.Cu") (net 3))
 (segment (start 77.919998 65.159999) (end 63.830001 65.159999) (width 1.5) (layer "F.Cu") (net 3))
 (segment (start 57.13 63.369999) (end 58.92 65.159999) (width 5) (layer "F.Cu") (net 21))
 (segment (start 57.13 60.15) (end 57.13 63.369999) (width 5) (layer "F.Cu") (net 21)))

